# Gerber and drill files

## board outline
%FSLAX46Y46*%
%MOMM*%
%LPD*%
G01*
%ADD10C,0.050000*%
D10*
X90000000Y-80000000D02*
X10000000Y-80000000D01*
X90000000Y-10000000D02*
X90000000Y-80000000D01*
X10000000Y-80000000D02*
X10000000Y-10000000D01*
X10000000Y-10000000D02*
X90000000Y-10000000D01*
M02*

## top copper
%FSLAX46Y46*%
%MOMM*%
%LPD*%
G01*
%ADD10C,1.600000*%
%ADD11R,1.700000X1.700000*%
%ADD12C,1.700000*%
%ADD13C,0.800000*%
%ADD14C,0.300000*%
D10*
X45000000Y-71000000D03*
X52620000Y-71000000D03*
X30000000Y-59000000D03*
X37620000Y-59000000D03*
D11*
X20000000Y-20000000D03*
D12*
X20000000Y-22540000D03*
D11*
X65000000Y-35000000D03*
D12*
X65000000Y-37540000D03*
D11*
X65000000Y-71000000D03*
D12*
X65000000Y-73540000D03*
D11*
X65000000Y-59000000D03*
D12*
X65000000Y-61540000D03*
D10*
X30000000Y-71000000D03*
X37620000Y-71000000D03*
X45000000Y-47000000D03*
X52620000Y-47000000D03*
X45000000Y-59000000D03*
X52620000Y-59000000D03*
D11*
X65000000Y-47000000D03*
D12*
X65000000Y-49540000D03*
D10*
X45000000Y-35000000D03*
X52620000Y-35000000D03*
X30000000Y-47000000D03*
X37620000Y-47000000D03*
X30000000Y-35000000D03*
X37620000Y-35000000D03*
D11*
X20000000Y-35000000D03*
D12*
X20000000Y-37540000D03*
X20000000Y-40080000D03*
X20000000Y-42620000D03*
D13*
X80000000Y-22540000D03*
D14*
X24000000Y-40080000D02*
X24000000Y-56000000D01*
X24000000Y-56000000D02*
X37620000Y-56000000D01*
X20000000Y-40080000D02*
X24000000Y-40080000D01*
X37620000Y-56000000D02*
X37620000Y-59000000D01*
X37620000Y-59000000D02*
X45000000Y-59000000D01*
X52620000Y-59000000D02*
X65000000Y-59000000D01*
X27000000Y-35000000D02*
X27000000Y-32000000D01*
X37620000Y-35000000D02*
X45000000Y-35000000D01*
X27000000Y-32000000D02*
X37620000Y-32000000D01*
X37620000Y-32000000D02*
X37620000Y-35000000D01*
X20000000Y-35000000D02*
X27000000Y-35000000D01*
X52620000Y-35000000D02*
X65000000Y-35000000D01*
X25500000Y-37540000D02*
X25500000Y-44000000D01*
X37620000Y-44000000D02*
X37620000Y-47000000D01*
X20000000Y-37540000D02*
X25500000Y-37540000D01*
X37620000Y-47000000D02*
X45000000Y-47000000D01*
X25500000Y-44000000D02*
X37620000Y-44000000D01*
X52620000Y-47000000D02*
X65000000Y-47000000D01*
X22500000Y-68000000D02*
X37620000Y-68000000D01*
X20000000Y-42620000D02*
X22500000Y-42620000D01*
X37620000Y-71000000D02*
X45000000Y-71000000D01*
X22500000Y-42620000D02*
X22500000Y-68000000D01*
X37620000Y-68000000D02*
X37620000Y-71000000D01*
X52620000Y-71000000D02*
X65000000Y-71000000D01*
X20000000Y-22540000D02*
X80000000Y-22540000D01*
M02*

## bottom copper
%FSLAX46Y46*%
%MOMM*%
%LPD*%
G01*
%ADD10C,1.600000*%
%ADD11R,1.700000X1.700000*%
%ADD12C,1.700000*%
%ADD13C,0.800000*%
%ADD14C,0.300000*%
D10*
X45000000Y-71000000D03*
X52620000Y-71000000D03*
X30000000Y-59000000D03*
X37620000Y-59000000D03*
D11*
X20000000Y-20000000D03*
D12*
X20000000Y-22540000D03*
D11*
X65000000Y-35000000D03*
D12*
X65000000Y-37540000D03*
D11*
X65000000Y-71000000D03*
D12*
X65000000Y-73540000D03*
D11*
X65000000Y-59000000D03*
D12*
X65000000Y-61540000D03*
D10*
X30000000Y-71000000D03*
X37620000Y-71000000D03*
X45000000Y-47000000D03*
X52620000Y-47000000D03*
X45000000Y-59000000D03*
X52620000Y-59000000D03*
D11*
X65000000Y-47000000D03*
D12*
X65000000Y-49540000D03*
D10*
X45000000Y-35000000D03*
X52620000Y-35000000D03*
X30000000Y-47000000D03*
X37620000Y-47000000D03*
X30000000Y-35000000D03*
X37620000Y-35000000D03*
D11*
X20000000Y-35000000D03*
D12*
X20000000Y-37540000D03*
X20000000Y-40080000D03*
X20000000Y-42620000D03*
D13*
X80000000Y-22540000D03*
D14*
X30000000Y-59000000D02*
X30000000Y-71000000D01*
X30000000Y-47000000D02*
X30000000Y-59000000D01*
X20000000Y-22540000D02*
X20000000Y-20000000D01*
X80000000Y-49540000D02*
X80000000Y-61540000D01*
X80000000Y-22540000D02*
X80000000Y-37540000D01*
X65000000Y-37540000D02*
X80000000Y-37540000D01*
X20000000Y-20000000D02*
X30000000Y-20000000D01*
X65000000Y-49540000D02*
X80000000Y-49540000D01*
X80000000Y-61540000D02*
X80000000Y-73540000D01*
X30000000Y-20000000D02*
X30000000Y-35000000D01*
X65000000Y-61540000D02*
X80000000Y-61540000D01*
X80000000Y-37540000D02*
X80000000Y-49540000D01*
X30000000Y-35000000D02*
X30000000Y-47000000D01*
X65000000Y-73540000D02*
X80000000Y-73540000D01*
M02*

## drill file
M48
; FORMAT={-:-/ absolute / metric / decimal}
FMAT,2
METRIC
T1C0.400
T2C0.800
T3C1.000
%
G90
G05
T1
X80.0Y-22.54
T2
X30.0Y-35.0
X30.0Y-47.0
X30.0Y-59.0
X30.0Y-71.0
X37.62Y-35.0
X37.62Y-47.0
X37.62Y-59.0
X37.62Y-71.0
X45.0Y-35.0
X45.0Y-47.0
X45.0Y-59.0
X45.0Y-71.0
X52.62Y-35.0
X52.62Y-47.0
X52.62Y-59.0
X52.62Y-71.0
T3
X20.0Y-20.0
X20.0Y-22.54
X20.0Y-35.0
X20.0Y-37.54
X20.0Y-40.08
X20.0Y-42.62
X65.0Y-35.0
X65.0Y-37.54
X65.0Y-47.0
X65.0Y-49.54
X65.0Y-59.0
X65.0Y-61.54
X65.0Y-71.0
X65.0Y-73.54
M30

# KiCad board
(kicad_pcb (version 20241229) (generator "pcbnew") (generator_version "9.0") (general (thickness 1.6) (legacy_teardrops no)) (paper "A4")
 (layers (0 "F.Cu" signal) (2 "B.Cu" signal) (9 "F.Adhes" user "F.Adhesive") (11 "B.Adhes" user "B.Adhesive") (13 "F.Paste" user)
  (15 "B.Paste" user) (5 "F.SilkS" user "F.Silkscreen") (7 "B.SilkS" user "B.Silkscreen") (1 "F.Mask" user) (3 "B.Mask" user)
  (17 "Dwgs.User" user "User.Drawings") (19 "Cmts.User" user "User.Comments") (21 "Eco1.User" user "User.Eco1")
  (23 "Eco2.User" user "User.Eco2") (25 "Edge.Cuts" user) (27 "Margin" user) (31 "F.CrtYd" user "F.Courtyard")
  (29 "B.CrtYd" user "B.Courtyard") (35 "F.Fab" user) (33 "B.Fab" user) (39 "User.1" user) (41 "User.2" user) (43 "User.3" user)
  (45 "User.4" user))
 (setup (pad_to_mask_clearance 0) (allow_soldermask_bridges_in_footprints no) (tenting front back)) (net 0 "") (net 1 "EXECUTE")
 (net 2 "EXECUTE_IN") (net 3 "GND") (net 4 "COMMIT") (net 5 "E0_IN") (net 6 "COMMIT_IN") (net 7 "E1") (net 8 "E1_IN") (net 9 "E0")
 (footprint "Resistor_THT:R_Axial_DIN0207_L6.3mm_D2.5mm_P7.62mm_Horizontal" (layer "F.Cu") (at 45 71)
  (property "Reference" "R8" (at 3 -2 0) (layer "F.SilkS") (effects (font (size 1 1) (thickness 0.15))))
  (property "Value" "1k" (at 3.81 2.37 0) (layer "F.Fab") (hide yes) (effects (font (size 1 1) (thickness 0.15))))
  (pad "1" thru_hole circle (at 0 0) (size 1.6 1.6) (drill 0.8) (layers "*.Cu" "*.Mask") (remove_unused_layers no) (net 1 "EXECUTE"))
  (pad "2" thru_hole circle (at 7.62 0) (size 1.6 1.6) (drill 0.8) (layers "*.Cu" "*.Mask") (remove_unused_layers no) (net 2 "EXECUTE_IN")))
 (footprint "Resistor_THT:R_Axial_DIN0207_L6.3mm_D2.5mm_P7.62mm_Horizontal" (layer "F.Cu") (at 30 59)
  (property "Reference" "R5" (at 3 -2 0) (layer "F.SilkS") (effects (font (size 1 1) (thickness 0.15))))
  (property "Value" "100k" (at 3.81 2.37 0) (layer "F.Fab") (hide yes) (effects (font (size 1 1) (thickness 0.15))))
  (pad "1" thru_hole circle (at 0 0) (size 1.6 1.6) (drill 0.8) (layers "*.Cu" "*.Mask") (remove_unused_layers no) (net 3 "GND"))
  (pad "2" thru_hole circle (at 7.62 0) (size 1.6 1.6) (drill 0.8) (layers "*.Cu" "*.Mask") (remove_unused_layers no) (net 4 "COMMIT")))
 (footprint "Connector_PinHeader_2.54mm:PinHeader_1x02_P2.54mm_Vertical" (layer "F.Cu") (at 20 20)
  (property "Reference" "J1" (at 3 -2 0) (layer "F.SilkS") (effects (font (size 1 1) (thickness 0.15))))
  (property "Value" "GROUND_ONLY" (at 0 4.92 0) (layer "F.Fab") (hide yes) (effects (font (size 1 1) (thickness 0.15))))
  (pad "1" thru_hole rect (at 0 0) (size 1.7 1.7) (drill 1) (layers "*.Cu" "*.Mask") (remove_unused_layers no) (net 3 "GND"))
  (pad "2" thru_hole circle (at 0 2.54) (size 1.7 1.7) (drill 1) (layers "*.Cu" "*.Mask") (remove_unused_layers no) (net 3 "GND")))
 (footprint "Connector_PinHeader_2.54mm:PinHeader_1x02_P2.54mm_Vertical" (layer "F.Cu") (at 65 35)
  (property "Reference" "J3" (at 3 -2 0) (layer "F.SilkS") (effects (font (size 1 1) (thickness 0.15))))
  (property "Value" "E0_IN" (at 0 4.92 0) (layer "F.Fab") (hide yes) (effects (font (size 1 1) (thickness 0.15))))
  (pad "1" thru_hole rect (at 0 0) (size 1.7 1.7) (drill 1) (layers "*.Cu" "*.Mask") (remove_unused_layers no) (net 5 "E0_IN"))
  (pad "2" thru_hole circle (at 0 2.54) (size 1.7 1.7) (drill 1) (layers "*.Cu" "*.Mask") (remove_unused_layers no) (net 3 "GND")))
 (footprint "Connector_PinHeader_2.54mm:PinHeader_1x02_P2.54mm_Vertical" (layer "F.Cu") (at 65 71)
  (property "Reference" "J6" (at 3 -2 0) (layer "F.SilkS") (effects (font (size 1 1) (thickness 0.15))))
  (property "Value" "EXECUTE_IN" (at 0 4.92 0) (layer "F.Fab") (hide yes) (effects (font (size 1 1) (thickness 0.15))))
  (pad "1" thru_hole rect (at 0 0) (size 1.7 1.7) (drill 1) (layers "*.Cu" "*.Mask") (remove_unused_layers no) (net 2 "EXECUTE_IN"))
  (pad "2" thru_hole circle (at 0 2.54) (size 1.7 1.7) (drill 1) (layers "*.Cu" "*.Mask") (remove_unused_layers no) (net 3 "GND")))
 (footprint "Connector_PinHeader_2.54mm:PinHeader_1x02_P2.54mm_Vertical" (layer "F.Cu") (at 65 59)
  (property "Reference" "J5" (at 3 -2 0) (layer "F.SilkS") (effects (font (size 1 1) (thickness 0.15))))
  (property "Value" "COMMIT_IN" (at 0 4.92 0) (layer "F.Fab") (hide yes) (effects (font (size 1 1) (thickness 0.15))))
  (pad "1" thru_hole rect (at 0 0) (size 1.7 1.7) (drill 1) (layers "*.Cu" "*.Mask") (remove_unused_layers no) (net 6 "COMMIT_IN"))
  (pad "2" thru_hole circle (at 0 2.54) (size 1.7 1.7) (drill 1) (layers "*.Cu" "*.Mask") (remove_unused_layers no) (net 3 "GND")))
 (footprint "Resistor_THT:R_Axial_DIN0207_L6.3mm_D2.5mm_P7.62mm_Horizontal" (layer "F.Cu") (at 30 71)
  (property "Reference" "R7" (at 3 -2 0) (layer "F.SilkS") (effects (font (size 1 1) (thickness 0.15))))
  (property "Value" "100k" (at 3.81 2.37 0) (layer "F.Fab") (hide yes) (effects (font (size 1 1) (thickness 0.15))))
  (pad "1" thru_hole circle (at 0 0) (size 1.6 1.6) (drill 0.8) (layers "*.Cu" "*.Mask") (remove_unused_layers no) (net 3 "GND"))
  (pad "2" thru_hole circle (at 7.62 0) (size 1.6 1.6) (drill 0.8) (layers "*.Cu" "*.Mask") (remove_unused_layers no) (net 1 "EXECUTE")))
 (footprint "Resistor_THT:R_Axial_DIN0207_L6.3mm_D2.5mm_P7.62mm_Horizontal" (layer "F.Cu") (at 45 47)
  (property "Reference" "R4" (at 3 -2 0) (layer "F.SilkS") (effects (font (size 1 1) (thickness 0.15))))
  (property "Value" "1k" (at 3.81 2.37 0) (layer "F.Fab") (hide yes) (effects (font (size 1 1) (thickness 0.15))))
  (pad "1" thru_hole circle (at 0 0) (size 1.6 1.6) (drill 0.8) (layers "*.Cu" "*.Mask") (remove_unused_layers no) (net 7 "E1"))
  (pad "2" thru_hole circle (at 7.62 0) (size 1.6 1.6) (drill 0.8) (layers "*.Cu" "*.Mask") (remove_unused_layers no) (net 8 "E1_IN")))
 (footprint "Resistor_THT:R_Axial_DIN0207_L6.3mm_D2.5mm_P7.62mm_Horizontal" (layer "F.Cu") (at 45 59)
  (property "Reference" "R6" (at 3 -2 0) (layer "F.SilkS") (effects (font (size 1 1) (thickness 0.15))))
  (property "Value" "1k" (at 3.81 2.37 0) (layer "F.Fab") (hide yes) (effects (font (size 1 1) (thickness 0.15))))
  (pad "1" thru_hole circle (at 0 0) (size 1.6 1.6) (drill 0.8) (layers "*.Cu" "*.Mask") (remove_unused_layers no) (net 4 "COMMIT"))
  (pad "2" thru_hole circle (at 7.62 0) (size 1.6 1.6) (drill 0.8) (layers "*.Cu" "*.Mask") (remove_unused_layers no) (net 6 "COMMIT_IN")))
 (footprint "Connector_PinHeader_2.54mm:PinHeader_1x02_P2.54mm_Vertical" (layer "F.Cu") (at 65 47)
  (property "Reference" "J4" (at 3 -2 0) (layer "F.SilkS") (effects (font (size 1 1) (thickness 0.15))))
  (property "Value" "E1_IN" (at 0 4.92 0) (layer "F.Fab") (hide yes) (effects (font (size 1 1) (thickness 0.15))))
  (pad "1" thru_hole rect (at 0 0) (size 1.7 1.7) (drill 1) (layers "*.Cu" "*.Mask") (remove_unused_layers no) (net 8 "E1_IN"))
  (pad "2" thru_hole circle (at 0 2.54) (size 1.7 1.7) (drill 1) (layers "*.Cu" "*.Mask") (remove_unused_layers no) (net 3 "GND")))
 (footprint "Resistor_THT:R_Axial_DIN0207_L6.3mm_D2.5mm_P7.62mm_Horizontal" (layer "F.Cu") (at 45 35)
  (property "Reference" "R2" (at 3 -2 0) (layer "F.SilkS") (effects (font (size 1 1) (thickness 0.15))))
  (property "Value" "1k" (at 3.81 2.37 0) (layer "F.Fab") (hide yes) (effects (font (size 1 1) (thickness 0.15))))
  (pad "1" thru_hole circle (at 0 0) (size 1.6 1.6) (drill 0.8) (layers "*.Cu" "*.Mask") (remove_unused_layers no) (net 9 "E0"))
  (pad "2" thru_hole circle (at 7.62 0) (size 1.6 1.6) (drill 0.8) (layers "*.Cu" "*.Mask") (remove_unused_layers no) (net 5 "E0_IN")))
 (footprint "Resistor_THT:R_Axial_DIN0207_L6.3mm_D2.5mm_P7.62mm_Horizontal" (layer "F.Cu") (at 30 47)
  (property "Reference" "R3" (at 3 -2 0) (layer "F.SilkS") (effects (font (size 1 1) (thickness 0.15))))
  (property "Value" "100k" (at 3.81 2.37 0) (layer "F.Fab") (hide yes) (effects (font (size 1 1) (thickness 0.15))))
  (pad "1" thru_hole circle (at 0 0) (size 1.6 1.6) (drill 0.8) (layers "*.Cu" "*.Mask") (remove_unused_layers no) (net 3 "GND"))
  (pad "2" thru_hole circle (at 7.62 0) (size 1.6 1.6) (drill 0.8) (layers "*.Cu" "*.Mask") (remove_unused_layers no) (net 7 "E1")))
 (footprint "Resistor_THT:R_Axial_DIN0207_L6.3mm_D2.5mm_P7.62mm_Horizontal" (layer "F.Cu") (at 30 35)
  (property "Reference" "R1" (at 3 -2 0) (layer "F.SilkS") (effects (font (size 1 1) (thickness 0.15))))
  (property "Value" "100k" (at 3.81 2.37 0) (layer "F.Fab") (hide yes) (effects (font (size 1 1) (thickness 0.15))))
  (pad "1" thru_hole circle (at 0 0) (size 1.6 1.6) (drill 0.8) (layers "*.Cu" "*.Mask") (remove_unused_layers no) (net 3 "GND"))
  (pad "2" thru_hole circle (at 7.62 0) (size 1.6 1.6) (drill 0.8) (layers "*.Cu" "*.Mask") (remove_unused_layers no) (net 9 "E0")))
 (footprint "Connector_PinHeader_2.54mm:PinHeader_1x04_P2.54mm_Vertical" (layer "F.Cu") (at 20 35)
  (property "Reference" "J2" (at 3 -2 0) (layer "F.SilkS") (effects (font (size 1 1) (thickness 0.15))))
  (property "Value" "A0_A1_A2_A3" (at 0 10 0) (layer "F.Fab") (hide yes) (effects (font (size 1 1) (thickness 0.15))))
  (pad "1" thru_hole rect (at 0 0) (size 1.7 1.7) (drill 1) (layers "*.Cu" "*.Mask") (remove_unused_layers no) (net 9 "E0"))
  (pad "2" thru_hole circle (at 0 2.54) (size 1.7 1.7) (drill 1) (layers "*.Cu" "*.Mask") (remove_unused_layers no) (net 7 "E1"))
  (pad "3" thru_hole circle (at 0 5.08) (size 1.7 1.7) (drill 1) (layers "*.Cu" "*.Mask") (remove_unused_layers no) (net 4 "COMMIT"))
  (pad "4" thru_hole circle (at 0 7.62) (size 1.7 1.7) (drill 1) (layers "*.Cu" "*.Mask") (remove_unused_layers no) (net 1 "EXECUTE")))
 (gr_line (start 90 80) (end 10 80) (stroke (width 0.05) (type default)) (layer "Edge.Cuts"))
 (gr_line (start 90 10) (end 90 80) (stroke (width 0.05) (type default)) (layer "Edge.Cuts"))
 (gr_line (start 10 80) (end 10 10) (stroke (width 0.05) (type default)) (layer "Edge.Cuts"))
 (gr_line (start 10 10) (end 90 10) (stroke (width 0.05) (type default)) (layer "Edge.Cuts"))
 (segment (start 24 40.08) (end 24 56) (width 0.3) (layer "F.Cu") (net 4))
 (segment (start 24 56) (end 37.62 56) (width 0.3) (layer "F.Cu") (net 4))
 (segment (start 20 40.08) (end 24 40.08) (width 0.3) (layer "F.Cu") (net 4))
 (segment (start 37.62 56) (end 37.62 59) (width 0.3) (layer "F.Cu") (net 4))
 (segment (start 37.62 59) (end 45 59) (width 0.3) (layer "F.Cu") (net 4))
 (segment (start 52.62 59) (end 65 59) (width 0.3) (layer "F.Cu") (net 6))
 (segment (start 27 35) (end 27 32) (width 0.3) (layer "F.Cu") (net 9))
 (segment (start 37.62 35) (end 45 35) (width 0.3) (layer "F.Cu") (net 9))
 (segment (start 27 32) (end 37.62 32) (width 0.3) (layer "F.Cu") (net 9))
 (segment (start 37.62 32) (end 37.62 35) (width 0.3) (layer "F.Cu") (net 9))
 (segment (start 20 35) (end 27 35) (width 0.3) (layer "F.Cu") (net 9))
 (segment (start 52.62 35) (end 65 35) (width 0.3) (layer "F.Cu") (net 5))
 (segment (start 25.5 37.54) (end 25.5 44) (width 0.3) (layer "F.Cu") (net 7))
 (segment (start 37.62 44) (end 37.62 47) (width 0.3) (layer "F.Cu") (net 7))
 (segment (start 20 37.54) (end 25.5 37.54) (width 0.3) (layer "F.Cu") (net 7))
 (segment (start 37.62 47) (end 45 47) (width 0.3) (layer "F.Cu") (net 7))
 (segment (start 25.5 44) (end 37.62 44) (width 0.3) (layer "F.Cu") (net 7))
 (segment (start 52.62 47) (end 65 47) (width 0.3) (layer "F.Cu") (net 8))
 (segment (start 22.5 68) (end 37.62 68) (width 0.3) (layer "F.Cu") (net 1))
 (segment (start 20 42.62) (end 22.5 42.62) (width 0.3) (layer "F.Cu") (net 1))
 (segment (start 37.62 71) (end 45 71) (width 0.3) (layer "F.Cu") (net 1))
 (segment (start 22.5 42.62) (end 22.5 68) (width 0.3) (layer "F.Cu") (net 1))
 (segment (start 37.62 68) (end 37.62 71) (width 0.3) (layer "F.Cu") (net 1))
 (segment (start 52.62 71) (end 65 71) (width 0.3) (layer "F.Cu") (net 2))
 (segment (start 20 22.54) (end 80 22.54) (width 0.3) (layer "F.Cu") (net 3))
 (via (at 80 22.54) (size 0.8) (drill 0.4) (layers "F.Cu" "B.Cu") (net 3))
 (segment (start 30 59) (end 30 71) (width 0.3) (layer "B.Cu") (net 3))
 (segment (start 30 47) (end 30 59) (width 0.3) (layer "B.Cu") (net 3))
 (segment (start 20 22.54) (end 20 20) (width 0.3) (layer "B.Cu") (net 3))
 (segment (start 80 49.54) (end 80 61.54) (width 0.3) (layer "B.Cu") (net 3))
 (segment (start 80 22.54) (end 80 37.54) (width 0.3) (layer "B.Cu") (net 3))
 (segment (start 65 37.54) (end 80 37.54) (width 0.3) (layer "B.Cu") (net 3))
 (segment (start 20 20) (end 30 20) (width 0.3) (layer "B.Cu") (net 3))
 (segment (start 65 49.54) (end 80 49.54) (width 0.3) (layer "B.Cu") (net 3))
 (segment (start 80 61.54) (end 80 73.54) (width 0.3) (layer "B.Cu") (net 3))
 (segment (start 30 20) (end 30 35) (width 0.3) (layer "B.Cu") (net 3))
 (segment (start 65 61.54) (end 80 61.54) (width 0.3) (layer "B.Cu") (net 3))
 (segment (start 80 37.54) (end 80 49.54) (width 0.3) (layer "B.Cu") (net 3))
 (segment (start 30 35) (end 30 47) (width 0.3) (layer "B.Cu") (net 3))
 (segment (start 65 73.54) (end 80 73.54) (width 0.3) (layer "B.Cu") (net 3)))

